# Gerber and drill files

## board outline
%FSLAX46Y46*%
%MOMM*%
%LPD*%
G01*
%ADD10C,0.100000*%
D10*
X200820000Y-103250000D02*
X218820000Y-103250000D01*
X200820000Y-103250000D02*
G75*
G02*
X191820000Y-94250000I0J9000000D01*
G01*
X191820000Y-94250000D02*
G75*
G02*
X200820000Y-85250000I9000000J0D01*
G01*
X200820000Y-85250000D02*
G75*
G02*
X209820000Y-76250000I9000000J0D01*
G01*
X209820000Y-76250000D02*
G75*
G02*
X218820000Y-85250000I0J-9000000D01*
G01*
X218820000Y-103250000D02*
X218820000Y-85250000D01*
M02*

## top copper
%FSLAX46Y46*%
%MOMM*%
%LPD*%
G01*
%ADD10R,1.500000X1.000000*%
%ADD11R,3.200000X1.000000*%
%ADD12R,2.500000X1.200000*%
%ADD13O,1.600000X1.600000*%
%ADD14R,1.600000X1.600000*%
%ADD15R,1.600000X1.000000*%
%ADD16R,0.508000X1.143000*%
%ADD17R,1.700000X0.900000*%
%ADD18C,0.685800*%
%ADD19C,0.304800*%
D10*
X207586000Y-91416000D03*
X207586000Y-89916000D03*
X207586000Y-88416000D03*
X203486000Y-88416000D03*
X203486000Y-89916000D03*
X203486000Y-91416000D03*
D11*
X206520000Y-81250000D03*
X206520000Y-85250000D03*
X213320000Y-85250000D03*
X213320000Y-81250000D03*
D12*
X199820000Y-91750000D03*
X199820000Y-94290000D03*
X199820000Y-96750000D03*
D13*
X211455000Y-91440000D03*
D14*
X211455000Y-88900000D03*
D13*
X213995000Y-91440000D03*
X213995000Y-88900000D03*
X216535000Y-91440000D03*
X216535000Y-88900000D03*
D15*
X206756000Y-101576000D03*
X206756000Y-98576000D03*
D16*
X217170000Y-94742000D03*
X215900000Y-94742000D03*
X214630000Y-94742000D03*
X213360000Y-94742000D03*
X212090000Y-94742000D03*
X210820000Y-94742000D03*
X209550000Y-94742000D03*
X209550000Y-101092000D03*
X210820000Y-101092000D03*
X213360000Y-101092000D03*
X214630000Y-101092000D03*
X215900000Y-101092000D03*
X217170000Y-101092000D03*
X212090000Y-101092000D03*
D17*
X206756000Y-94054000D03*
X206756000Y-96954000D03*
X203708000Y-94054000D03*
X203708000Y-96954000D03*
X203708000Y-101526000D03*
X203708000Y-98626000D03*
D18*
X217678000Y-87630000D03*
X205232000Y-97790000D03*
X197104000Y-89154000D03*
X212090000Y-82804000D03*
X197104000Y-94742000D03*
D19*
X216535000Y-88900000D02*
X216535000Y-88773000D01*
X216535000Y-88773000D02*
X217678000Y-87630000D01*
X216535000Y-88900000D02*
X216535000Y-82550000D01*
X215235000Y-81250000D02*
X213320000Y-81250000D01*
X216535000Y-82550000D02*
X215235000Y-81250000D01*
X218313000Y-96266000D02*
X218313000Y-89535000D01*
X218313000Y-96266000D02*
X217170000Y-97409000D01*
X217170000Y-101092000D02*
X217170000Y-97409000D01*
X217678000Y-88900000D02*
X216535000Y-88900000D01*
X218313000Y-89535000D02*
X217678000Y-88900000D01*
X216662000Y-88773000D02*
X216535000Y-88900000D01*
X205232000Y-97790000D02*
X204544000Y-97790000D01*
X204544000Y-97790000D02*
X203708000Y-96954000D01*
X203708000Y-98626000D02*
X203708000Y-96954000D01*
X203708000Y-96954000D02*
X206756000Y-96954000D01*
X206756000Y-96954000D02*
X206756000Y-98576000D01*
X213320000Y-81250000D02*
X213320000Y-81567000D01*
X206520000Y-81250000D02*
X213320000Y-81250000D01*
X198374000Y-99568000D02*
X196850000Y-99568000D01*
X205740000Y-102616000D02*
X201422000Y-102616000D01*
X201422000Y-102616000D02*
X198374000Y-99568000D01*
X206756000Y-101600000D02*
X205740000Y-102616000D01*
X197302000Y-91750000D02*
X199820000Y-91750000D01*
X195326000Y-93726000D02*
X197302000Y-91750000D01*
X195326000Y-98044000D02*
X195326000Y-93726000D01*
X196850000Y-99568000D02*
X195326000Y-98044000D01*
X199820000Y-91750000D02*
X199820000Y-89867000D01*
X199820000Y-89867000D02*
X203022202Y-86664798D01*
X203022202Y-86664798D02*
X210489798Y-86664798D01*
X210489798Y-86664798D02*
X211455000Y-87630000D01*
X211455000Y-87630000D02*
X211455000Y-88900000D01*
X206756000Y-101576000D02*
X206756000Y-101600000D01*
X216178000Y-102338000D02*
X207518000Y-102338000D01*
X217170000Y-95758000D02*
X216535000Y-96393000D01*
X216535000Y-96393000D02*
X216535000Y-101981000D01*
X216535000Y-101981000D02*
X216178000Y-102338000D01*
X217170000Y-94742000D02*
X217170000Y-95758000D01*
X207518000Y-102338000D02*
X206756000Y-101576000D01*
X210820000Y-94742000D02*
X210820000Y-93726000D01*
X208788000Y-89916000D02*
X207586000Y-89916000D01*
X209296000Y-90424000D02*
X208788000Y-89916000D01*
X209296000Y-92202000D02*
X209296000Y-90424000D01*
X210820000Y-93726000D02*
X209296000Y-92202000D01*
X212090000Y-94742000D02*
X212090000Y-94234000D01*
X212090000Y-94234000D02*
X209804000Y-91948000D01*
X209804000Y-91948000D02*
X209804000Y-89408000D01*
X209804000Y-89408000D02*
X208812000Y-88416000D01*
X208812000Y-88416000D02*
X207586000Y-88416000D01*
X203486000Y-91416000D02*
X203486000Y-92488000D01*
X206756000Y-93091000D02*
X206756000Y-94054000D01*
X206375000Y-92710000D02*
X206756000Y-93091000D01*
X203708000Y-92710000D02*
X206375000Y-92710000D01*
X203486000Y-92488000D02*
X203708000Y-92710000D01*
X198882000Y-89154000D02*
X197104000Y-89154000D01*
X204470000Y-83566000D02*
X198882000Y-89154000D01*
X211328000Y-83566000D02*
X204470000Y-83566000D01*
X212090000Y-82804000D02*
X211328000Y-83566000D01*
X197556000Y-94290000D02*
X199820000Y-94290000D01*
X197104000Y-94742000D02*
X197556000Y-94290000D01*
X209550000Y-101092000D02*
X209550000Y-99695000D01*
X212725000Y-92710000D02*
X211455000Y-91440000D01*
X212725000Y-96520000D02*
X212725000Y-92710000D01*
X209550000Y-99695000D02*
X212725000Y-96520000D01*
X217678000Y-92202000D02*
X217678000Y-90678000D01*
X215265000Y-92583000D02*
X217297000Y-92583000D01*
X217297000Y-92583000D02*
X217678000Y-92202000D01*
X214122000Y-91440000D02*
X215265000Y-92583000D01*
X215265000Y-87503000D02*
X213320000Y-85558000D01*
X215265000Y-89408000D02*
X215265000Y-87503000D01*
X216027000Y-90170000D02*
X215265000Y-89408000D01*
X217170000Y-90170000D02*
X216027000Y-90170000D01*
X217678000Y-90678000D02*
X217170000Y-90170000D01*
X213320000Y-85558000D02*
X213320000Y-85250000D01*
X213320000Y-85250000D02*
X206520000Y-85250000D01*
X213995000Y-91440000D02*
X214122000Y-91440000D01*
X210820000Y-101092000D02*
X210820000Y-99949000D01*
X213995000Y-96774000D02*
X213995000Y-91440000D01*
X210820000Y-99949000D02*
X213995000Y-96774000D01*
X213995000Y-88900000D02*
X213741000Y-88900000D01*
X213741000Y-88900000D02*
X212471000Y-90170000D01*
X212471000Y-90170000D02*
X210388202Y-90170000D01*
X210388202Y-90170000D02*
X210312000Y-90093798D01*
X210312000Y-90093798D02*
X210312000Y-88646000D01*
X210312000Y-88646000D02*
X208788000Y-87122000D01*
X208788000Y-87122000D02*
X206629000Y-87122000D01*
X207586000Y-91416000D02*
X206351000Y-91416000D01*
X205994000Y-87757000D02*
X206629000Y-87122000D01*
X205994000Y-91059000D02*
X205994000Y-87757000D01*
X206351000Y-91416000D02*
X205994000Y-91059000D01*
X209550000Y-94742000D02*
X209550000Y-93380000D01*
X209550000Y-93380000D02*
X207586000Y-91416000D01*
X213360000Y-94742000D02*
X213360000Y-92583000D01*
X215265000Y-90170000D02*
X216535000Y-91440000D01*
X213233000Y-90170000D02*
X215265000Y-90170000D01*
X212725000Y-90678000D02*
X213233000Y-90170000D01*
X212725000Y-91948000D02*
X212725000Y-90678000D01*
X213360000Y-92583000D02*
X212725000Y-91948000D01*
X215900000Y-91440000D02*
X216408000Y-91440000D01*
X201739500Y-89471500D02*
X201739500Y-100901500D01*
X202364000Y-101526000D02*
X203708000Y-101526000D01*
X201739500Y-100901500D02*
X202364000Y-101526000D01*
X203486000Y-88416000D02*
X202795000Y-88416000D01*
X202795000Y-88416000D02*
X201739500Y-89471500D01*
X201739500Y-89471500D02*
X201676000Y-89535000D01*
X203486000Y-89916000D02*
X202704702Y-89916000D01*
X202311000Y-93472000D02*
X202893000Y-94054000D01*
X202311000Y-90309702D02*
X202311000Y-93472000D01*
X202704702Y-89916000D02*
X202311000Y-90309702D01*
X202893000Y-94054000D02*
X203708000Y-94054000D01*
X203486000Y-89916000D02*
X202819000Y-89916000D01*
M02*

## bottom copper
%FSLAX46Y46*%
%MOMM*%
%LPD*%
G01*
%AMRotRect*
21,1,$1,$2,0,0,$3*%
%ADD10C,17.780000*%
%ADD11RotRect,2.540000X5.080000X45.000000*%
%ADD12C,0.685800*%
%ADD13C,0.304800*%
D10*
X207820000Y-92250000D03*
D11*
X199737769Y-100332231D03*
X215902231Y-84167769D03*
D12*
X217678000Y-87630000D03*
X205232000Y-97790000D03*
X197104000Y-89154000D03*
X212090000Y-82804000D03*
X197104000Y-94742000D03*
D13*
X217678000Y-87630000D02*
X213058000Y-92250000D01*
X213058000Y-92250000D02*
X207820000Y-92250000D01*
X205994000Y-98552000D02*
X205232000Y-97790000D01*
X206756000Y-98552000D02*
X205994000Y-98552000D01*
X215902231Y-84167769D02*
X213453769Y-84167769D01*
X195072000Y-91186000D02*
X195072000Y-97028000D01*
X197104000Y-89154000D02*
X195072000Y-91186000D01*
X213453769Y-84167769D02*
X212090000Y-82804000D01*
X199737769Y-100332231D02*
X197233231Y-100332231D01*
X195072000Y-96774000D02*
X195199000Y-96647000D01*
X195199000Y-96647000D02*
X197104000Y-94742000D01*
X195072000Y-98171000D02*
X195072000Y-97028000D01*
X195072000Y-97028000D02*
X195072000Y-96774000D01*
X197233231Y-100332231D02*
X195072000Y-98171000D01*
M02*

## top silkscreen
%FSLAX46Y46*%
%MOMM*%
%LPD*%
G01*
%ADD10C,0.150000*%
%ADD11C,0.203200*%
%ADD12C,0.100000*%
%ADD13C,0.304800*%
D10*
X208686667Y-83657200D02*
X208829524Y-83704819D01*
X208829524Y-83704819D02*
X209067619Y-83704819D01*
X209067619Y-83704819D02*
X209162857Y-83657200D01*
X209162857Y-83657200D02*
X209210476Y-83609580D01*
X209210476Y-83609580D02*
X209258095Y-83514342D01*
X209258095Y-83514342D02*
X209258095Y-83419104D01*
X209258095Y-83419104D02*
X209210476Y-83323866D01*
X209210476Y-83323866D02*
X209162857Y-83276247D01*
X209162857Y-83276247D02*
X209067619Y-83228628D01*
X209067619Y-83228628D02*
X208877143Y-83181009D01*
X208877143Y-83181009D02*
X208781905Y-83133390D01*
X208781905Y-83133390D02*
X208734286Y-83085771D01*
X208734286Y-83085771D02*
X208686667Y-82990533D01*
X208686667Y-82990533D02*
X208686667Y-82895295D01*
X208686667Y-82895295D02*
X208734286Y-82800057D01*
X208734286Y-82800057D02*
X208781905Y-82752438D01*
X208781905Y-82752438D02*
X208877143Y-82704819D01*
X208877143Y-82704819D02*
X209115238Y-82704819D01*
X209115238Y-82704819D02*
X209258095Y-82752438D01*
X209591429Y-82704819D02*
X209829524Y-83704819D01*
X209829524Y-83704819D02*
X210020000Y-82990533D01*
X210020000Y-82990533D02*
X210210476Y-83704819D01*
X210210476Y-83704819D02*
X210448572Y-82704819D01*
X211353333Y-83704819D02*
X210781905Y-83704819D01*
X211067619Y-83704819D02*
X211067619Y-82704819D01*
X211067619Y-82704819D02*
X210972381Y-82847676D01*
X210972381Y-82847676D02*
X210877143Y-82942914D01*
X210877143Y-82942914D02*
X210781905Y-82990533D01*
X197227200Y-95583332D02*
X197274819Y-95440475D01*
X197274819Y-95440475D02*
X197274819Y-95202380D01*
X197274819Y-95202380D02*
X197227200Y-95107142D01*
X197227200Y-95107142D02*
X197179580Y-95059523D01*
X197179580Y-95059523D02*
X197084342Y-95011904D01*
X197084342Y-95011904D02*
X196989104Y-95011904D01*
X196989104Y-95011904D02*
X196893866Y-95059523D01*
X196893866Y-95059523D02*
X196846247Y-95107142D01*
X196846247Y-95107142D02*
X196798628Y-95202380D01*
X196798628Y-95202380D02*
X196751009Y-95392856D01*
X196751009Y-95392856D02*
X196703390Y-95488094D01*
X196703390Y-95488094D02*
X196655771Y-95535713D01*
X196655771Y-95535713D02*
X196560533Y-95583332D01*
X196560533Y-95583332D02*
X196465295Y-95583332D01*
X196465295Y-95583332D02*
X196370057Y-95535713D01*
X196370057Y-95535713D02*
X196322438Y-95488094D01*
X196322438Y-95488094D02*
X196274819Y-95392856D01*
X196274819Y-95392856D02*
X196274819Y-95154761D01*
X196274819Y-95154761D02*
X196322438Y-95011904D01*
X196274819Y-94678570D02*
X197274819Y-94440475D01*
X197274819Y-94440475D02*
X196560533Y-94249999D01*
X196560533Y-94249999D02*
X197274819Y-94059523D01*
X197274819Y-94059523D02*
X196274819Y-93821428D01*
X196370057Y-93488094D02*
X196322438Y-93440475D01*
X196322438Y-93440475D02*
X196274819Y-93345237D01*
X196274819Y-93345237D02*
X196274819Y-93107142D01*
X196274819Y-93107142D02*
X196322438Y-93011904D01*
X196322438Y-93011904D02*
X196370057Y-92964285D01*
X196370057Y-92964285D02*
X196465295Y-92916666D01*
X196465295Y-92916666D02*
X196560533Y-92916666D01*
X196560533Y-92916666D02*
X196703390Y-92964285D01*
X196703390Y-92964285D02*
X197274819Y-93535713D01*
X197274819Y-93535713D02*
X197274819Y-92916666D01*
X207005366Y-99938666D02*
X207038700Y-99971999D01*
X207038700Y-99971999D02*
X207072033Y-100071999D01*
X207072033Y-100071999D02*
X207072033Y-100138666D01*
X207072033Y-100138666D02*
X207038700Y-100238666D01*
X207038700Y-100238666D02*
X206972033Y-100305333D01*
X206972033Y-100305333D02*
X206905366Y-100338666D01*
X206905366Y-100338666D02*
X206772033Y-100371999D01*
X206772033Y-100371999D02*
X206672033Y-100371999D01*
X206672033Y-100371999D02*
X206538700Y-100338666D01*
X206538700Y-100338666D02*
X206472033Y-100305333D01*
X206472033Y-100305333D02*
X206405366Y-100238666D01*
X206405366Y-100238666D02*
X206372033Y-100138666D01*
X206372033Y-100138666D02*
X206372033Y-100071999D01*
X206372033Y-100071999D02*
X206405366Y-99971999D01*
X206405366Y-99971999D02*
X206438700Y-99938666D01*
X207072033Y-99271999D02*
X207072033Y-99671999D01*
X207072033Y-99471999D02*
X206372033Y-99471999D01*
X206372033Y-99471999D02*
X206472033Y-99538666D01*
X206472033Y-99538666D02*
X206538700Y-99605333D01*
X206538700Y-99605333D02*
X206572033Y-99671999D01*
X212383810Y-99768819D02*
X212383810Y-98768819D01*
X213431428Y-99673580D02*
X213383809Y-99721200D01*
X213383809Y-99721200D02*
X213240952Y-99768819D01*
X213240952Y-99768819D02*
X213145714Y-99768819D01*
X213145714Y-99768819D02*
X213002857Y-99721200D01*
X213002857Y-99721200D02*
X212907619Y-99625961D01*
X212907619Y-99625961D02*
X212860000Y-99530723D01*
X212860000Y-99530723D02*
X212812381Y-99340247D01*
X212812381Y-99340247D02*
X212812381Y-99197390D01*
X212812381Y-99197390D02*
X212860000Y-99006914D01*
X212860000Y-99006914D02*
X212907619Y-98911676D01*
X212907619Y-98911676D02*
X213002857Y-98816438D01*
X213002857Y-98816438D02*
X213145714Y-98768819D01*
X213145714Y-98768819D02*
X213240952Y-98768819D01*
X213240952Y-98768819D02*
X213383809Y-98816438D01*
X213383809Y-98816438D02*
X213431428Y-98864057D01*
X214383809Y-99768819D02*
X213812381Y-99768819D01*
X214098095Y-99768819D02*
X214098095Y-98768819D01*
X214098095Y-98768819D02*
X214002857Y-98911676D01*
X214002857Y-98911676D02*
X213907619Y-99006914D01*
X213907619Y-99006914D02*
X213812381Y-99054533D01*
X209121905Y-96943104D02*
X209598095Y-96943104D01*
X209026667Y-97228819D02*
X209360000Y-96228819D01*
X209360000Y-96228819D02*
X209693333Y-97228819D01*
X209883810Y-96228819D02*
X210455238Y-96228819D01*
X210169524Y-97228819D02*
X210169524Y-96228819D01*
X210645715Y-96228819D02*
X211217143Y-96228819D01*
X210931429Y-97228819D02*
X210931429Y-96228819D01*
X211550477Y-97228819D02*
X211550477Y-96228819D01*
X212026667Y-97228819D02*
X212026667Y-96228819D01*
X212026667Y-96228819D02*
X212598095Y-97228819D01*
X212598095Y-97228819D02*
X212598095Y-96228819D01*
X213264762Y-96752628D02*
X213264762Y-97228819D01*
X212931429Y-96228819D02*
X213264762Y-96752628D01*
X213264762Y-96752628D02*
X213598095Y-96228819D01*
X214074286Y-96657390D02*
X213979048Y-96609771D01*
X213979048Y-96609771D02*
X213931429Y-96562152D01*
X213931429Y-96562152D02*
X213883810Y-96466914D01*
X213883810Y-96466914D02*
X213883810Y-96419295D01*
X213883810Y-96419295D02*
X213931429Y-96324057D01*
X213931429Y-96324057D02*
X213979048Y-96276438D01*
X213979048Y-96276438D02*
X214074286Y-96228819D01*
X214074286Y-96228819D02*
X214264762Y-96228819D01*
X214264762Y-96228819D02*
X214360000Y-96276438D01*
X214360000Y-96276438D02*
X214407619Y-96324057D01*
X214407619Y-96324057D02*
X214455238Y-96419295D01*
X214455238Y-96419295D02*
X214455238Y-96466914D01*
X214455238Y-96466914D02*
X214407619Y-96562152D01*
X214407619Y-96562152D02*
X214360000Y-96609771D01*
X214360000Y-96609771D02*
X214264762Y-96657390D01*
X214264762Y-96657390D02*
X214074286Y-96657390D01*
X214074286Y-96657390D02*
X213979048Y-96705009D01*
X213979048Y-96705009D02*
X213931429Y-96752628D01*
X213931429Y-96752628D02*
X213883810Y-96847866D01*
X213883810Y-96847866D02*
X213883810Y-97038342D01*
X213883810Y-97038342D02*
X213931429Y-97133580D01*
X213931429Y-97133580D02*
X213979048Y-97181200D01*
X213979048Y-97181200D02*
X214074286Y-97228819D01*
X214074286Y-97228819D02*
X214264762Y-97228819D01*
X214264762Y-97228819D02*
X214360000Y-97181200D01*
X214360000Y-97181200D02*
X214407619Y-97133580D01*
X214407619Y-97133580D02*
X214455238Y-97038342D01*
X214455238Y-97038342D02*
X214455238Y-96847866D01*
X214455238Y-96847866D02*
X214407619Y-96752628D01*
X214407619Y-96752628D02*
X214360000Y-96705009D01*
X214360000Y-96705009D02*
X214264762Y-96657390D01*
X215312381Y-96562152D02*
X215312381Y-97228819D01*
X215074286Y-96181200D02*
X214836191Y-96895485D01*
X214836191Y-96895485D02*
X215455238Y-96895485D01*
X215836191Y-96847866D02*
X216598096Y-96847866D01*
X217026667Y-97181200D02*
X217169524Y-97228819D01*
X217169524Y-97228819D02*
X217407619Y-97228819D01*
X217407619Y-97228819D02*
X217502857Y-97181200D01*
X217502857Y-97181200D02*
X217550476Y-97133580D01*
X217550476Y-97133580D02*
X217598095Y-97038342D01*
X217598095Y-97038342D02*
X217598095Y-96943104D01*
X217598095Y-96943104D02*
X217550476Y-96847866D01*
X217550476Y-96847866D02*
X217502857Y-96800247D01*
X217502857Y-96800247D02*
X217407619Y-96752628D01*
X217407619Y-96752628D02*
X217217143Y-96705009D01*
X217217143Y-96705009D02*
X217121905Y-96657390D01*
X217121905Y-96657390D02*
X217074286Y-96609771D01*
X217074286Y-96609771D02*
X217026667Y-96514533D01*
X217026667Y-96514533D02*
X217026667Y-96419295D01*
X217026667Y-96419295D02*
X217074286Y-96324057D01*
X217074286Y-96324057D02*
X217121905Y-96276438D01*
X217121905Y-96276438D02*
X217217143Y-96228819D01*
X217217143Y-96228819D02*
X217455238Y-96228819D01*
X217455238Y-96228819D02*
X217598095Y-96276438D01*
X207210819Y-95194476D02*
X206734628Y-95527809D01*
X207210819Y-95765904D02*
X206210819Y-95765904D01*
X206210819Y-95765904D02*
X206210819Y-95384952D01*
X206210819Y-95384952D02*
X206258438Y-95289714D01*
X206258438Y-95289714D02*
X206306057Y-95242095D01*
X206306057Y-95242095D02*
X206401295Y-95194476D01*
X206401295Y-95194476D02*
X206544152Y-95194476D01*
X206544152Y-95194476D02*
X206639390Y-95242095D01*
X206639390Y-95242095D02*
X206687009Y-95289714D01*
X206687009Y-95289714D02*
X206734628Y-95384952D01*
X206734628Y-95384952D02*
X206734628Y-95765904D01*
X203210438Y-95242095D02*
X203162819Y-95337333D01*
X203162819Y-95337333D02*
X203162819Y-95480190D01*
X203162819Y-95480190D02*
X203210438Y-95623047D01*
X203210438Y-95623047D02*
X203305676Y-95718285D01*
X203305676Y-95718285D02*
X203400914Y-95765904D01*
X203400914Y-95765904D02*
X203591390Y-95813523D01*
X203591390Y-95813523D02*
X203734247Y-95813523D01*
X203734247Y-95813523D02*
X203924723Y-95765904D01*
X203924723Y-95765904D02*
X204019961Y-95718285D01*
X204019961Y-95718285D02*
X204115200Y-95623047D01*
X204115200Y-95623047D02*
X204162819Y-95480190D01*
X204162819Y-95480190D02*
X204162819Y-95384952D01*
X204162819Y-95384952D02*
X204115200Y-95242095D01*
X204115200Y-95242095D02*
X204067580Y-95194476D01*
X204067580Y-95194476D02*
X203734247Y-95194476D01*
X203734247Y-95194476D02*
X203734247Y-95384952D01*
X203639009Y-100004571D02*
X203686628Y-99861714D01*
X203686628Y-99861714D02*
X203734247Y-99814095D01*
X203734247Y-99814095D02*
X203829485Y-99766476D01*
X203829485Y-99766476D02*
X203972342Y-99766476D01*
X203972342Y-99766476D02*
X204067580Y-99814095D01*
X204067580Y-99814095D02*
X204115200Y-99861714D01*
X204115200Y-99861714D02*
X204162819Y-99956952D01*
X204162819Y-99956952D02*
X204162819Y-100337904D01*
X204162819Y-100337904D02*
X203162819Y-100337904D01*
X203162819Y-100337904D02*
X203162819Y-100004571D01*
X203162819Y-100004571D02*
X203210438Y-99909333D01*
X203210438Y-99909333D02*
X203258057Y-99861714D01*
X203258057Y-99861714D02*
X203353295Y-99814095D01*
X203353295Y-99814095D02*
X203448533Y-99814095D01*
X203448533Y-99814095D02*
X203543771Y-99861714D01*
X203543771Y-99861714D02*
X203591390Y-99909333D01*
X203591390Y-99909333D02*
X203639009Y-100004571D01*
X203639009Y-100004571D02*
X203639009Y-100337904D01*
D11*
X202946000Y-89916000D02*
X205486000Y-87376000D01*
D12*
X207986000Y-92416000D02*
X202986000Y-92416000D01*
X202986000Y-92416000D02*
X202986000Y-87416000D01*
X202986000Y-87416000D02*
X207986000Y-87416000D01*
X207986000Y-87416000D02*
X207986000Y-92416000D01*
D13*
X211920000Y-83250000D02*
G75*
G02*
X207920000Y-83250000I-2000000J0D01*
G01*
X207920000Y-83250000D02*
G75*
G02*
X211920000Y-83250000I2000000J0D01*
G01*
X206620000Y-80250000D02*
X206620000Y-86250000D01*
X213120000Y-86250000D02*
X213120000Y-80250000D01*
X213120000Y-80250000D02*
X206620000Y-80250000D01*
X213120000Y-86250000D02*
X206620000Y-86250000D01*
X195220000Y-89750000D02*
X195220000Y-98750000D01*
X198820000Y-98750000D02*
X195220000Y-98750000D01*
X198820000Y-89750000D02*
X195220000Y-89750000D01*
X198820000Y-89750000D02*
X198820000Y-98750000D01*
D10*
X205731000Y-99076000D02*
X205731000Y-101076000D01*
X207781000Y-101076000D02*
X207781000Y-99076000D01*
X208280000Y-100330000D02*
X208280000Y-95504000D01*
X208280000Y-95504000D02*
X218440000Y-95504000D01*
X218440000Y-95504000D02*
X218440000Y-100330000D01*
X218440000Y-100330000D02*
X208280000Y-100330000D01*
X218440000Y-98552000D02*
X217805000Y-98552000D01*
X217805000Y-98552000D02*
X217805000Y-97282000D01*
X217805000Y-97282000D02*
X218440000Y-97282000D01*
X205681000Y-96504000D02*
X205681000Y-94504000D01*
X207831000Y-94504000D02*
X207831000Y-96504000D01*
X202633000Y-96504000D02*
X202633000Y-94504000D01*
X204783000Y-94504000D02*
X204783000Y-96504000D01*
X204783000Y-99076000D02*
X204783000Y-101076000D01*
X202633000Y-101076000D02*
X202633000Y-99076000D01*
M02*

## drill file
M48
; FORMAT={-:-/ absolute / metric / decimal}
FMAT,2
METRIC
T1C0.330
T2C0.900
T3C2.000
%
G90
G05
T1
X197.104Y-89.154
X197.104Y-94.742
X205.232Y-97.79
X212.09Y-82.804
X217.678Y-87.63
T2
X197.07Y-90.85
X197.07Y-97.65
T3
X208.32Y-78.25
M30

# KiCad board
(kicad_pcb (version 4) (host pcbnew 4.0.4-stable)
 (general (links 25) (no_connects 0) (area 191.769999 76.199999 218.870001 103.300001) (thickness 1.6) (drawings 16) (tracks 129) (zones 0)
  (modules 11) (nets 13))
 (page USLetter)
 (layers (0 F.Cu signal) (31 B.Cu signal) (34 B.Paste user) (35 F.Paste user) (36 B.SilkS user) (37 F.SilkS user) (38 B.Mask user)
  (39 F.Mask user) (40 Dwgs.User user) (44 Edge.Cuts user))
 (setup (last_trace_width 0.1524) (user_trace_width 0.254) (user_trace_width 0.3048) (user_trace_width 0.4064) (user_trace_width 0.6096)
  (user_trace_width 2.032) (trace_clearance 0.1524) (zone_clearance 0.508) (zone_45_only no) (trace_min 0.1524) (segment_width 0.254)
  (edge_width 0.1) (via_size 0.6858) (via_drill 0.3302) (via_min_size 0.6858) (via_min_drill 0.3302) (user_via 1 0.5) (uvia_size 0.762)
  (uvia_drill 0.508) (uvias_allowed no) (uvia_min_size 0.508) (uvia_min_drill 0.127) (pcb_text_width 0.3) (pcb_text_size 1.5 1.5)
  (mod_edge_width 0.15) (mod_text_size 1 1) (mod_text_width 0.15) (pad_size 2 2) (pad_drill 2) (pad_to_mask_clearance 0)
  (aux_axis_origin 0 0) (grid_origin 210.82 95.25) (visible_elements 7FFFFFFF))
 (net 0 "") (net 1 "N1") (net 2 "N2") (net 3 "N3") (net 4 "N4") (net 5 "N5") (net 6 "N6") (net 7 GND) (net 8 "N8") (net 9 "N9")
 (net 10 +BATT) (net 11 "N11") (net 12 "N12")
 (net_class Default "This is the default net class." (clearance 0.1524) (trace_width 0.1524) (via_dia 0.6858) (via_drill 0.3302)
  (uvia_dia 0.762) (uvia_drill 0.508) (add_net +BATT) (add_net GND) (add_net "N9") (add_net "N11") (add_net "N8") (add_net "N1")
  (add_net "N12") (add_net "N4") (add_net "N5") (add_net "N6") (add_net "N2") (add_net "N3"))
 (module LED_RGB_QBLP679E (layer F.Cu) (at 205.486 89.916 180)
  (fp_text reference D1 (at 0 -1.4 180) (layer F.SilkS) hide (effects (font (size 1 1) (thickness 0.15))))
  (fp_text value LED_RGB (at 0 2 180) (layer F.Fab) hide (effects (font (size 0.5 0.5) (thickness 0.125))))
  (fp_line (start 2.54 0) (end 0 2.54) (layer F.SilkS) (width 0.2032))
  (fp_line (start -2.5 -2.5) (end 2.5 -2.5) (layer F.SilkS) (width 0.1))
  (fp_line (start 2.5 -2.5) (end 2.5 2.5) (layer F.SilkS) (width 0.1))
  (fp_line (start 2.5 2.5) (end -2.5 2.5) (layer F.SilkS) (width 0.1))
  (fp_line (start -2.5 2.5) (end -2.5 -2.5) (layer F.SilkS) (width 0.1))
  (pad 4 smd rect (at -2.1 -1.5 270) (size 1 1.5) (layers F.Cu F.Paste F.Mask) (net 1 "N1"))
  (pad 5 smd rect (at -2.1 0 270) (size 1 1.5) (layers F.Cu F.Paste F.Mask) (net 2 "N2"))
  (pad 6 smd rect (at -2.1 1.5 270) (size 1 1.5) (layers F.Cu F.Paste F.Mask) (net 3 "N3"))
  (pad 1 smd rect (at 2 1.5 270) (size 1 1.5) (layers F.Cu F.Paste F.Mask) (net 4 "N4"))
  (pad 2 smd rect (at 2 0 270) (size 1 1.5) (layers F.Cu F.Paste F.Mask) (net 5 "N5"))
  (pad 3 smd rect (at 2 -1.5 270) (size 1 1.5) (layers F.Cu F.Paste F.Mask) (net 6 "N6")))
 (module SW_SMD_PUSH (layer F.Cu) (at 213.32 85.25 180)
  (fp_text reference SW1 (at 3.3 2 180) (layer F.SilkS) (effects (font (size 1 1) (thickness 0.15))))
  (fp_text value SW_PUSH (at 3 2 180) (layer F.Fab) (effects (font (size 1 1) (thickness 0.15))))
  (fp_circle (center 3.4 2) (end 3.4 0) (layer F.SilkS) (width 0.3048))
  (fp_line (start 6.7 5) (end 6.7 -1) (layer F.SilkS) (width 0.3048))
  (fp_line (start 0.2 -1) (end 0.2 5) (layer F.SilkS) (width 0.3048))
  (fp_line (start 0.2 5) (end 6.7 5) (layer F.SilkS) (width 0.3048))
  (fp_line (start 0.2 -1) (end 6.7 -1) (layer F.SilkS) (width 0.3048))
  (pad 2 smd rect (at 6.8 4 180) (size 3.2 1) (layers F.Cu F.Paste F.Mask) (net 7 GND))
  (pad 1 smd rect (at 6.8 0 180) (size 3.2 1) (layers F.Cu F.Paste F.Mask) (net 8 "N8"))
  (pad 1 smd rect (at 0 0 180) (size 3.2 1) (layers F.Cu F.Paste F.Mask) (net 8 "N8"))
  (pad 2 smd rect (at 0 4 180) (size 3.2 1) (layers F.Cu F.Paste F.Mask) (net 7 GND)))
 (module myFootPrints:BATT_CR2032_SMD (layer B.Cu) (at 207.82 92.25 45)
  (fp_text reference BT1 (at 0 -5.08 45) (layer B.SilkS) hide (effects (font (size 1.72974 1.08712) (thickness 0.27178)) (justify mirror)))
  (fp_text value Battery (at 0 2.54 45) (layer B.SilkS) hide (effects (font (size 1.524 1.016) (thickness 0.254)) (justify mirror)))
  (pad 2 smd circle (at 0 0 45) (size 17.78 17.78) (layers B.Cu B.Paste B.Mask) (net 7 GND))
  (pad 1 smd rect (at -11.43 0 45) (size 2.54 5.08) (layers B.Cu B.Paste B.Mask) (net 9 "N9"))
  (pad 1 smd rect (at 11.43 0 45) (size 2.54 5.08) (layers B.Cu B.Paste B.Mask) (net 9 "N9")))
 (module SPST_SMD (layer F.Cu) (at 199.82 94.25 270)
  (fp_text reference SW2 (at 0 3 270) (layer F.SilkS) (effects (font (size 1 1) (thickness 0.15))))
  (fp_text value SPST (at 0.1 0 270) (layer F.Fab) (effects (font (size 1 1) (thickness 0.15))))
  (fp_line (start -4.5 4.6) (end 4.5 4.6) (layer F.SilkS) (width 0.3048))
  (fp_line (start 4.5 1) (end 4.5 4.6) (layer F.SilkS) (width 0.3048))
  (fp_line (start -4.5 1) (end -4.5 4.6) (layer F.SilkS) (width 0.3048))
  (fp_line (start -4.5 1) (end 4.5 1) (layer F.SilkS) (width 0.3048))
  (pad "" np_thru_hole circle (at 3.4 2.75 270) (size 0.9 0.9) (drill 0.9) (layers *.Cu *.Mask))
  (pad 1 smd rect (at -2.5 0 270) (size 1.2 2.5) (layers F.Cu F.Paste F.Mask) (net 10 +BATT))
  (pad 2 smd rect (at 0.04 0 270) (size 1.2 2.5) (layers F.Cu F.Paste F.Mask) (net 9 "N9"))
  (pad 3 smd rect (at 2.5 0 270) (size 1.2 2.5) (layers F.Cu F.Paste F.Mask))
  (pad "" np_thru_hole circle (at -3.4 2.75 270) (size 0.9 0.9) (drill 0.9) (layers *.Cu *.Mask)))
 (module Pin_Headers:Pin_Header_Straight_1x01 (layer F.Cu) (at 208.32 78.25)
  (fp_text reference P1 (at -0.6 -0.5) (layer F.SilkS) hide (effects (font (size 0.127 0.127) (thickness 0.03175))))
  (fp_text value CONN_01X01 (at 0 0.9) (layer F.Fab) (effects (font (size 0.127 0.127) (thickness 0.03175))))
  (pad "" np_thru_hole circle (at 0 0) (size 2 2) (drill 2) (layers *.Cu *.Mask)))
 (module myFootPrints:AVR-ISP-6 (layer F.Cu) (at 211.455 91.44 90)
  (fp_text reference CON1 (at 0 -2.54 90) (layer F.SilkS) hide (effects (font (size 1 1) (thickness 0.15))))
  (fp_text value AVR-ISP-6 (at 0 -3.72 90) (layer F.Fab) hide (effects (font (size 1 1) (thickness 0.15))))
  (pad 1 smd oval (at 0 0 90) (size 1.6 1.6) (layers F.Cu F.Paste F.Mask) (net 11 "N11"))
  (pad 2 smd rect (at 2.54 0 90) (size 1.6 1.6) (layers F.Cu F.Paste F.Mask) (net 10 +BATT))
  (pad 3 smd oval (at 0 2.54 90) (size 1.6 1.6) (layers F.Cu F.Paste F.Mask) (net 8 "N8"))
  (pad 4 smd oval (at 2.54 2.54 90) (size 1.6 1.6) (layers F.Cu F.Paste F.Mask) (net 1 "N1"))
  (pad 5 smd oval (at 0 5.08 90) (size 1.6 1.6) (layers F.Cu F.Paste F.Mask) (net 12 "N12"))
  (pad 6 smd oval (at 2.54 5.08 90) (size 1.6 1.6) (layers F.Cu F.Paste F.Mask) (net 7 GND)))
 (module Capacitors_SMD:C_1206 (layer F.Cu) (at 206.756 100.076 90)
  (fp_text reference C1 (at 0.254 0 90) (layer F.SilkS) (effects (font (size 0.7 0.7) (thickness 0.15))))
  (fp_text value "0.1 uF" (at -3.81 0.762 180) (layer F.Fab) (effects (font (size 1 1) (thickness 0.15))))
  (fp_line (start 1 -1.025) (end -1 -1.025) (layer F.SilkS) (width 0.15))
  (fp_line (start -1 1.025) (end 1 1.025) (layer F.SilkS) (width 0.15))
  (pad 1 smd rect (at -1.5 0 90) (size 1 1.6) (layers F.Cu F.Paste F.Mask) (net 10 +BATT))
  (pad 2 smd rect (at 1.5 0 90) (size 1 1.6) (layers F.Cu F.Paste F.Mask) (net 7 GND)))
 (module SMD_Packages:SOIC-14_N (layer F.Cu) (at 213.36 98.044 180)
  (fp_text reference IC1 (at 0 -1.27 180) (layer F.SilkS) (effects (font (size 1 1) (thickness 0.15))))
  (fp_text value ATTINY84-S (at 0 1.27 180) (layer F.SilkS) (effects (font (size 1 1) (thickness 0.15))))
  (fp_line (start 5.08 -2.286) (end 5.08 2.54) (layer F.SilkS) (width 0.15))
  (fp_line (start 5.08 2.54) (end -5.08 2.54) (layer F.SilkS) (width 0.15))
  (fp_line (start -5.08 2.54) (end -5.08 -2.286) (layer F.SilkS) (width 0.15))
  (fp_line (start -5.08 -2.286) (end 5.08 -2.286) (layer F.SilkS) (width 0.15))
  (fp_line (start -5.08 -0.508) (end -4.445 -0.508) (layer F.SilkS) (width 0.15))
  (fp_line (start -4.445 -0.508) (end -4.445 0.762) (layer F.SilkS) (width 0.15))
  (fp_line (start -4.445 0.762) (end -5.08 0.762) (layer F.SilkS) (width 0.15))
  (pad 1 smd rect (at -3.81 3.302 180) (size 0.508 1.143) (layers F.Cu F.Paste F.Mask) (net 10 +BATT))
  (pad 2 smd rect (at -2.54 3.302 180) (size 0.508 1.143) (layers F.Cu F.Paste F.Mask))
  (pad 3 smd rect (at -1.27 3.302 180) (size 0.508 1.143) (layers F.Cu F.Paste F.Mask))
  (pad 4 smd rect (at 0 3.302 180) (size 0.508 1.143) (layers F.Cu F.Paste F.Mask) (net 12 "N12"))
  (pad 5 smd rect (at 1.27 3.302 180) (size 0.508 1.143) (layers F.Cu F.Paste F.Mask) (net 3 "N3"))
  (pad 6 smd rect (at 2.54 3.302 180) (size 0.508 1.143) (layers F.Cu F.Paste F.Mask) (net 2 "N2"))
  (pad 7 smd rect (at 3.81 3.302 180) (size 0.508 1.143) (layers F.Cu F.Paste F.Mask) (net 1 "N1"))
  (pad 8 smd rect (at 3.81 -3.048 180) (size 0.508 1.143) (layers F.Cu F.Paste F.Mask) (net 11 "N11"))
  (pad 9 smd rect (at 2.54 -3.048 180) (size 0.508 1.143) (layers F.Cu F.Paste F.Mask) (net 8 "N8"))
  (pad 11 smd rect (at 0 -3.048 180) (size 0.508 1.143) (layers F.Cu F.Paste F.Mask))
  (pad 12 smd rect (at -1.27 -3.048 180) (size 0.508 1.143) (layers F.Cu F.Paste F.Mask))
  (pad 13 smd rect (at -2.54 -3.048 180) (size 0.508 1.143) (layers F.Cu F.Paste F.Mask))
  (pad 14 smd rect (at -3.81 -3.048 180) (size 0.508 1.143) (layers F.Cu F.Paste F.Mask) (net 7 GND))
  (pad 10 smd rect (at 1.27 -3.048 180) (size 0.508 1.143) (layers F.Cu F.Paste F.Mask)))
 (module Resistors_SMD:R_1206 (layer F.Cu) (at 206.756 95.504 270)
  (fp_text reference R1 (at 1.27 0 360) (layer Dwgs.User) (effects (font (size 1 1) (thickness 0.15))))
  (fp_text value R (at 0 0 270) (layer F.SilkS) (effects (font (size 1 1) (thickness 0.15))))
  (fp_line (start 1 1.075) (end -1 1.075) (layer F.SilkS) (width 0.15))
  (fp_line (start -1 -1.075) (end 1 -1.075) (layer F.SilkS) (width 0.15))
  (pad 1 smd rect (at -1.45 0 270) (size 0.9 1.7) (layers F.Cu F.Paste F.Mask) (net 6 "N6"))
  (pad 2 smd rect (at 1.45 0 270) (size 0.9 1.7) (layers F.Cu F.Paste F.Mask) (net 7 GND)))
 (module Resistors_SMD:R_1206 (layer F.Cu) (at 203.708 95.504 270)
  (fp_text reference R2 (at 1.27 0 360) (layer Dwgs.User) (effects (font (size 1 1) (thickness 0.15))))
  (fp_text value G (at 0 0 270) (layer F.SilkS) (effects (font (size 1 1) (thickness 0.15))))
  (fp_line (start 1 1.075) (end -1 1.075) (layer F.SilkS) (width 0.15))
  (fp_line (start -1 -1.075) (end 1 -1.075) (layer F.SilkS) (width 0.15))
  (pad 1 smd rect (at -1.45 0 270) (size 0.9 1.7) (layers F.Cu F.Paste F.Mask) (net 5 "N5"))
  (pad 2 smd rect (at 1.45 0 270) (size 0.9 1.7) (layers F.Cu F.Paste F.Mask) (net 7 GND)))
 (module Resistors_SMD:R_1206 (layer F.Cu) (at 203.708 100.076 90)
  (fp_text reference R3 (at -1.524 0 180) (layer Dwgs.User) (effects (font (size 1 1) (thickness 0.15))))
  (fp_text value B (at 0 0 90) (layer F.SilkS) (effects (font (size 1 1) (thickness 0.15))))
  (fp_line (start 1 1.075) (end -1 1.075) (layer F.SilkS) (width 0.15))
  (fp_line (start -1 -1.075) (end 1 -1.075) (layer F.SilkS) (width 0.15))
  (pad 1 smd rect (at -1.45 0 90) (size 0.9 1.7) (layers F.Cu F.Paste F.Mask) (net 4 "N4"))
  (pad 2 smd rect (at 1.45 0 90) (size 0.9 1.7) (layers F.Cu F.Paste F.Mask) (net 7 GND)))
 (gr_line (start 200.82 103.25) (end 218.82 103.25) (angle 90) (layer Edge.Cuts) (width 0.1))
 (gr_arc (start 200.82 94.25) (end 200.82 103.25) (angle 90) (layer Edge.Cuts) (width 0.1))
 (gr_arc (start 200.82 94.25) (end 191.82 94.25) (angle 90) (layer Edge.Cuts) (width 0.1))
 (gr_arc (start 209.82 85.25) (end 200.82 85.25) (angle 90) (layer Edge.Cuts) (width 0.1))
 (gr_arc (start 209.82 85.25) (end 209.82 76.25) (angle 90) (layer Edge.Cuts) (width 0.1))
 (gr_line (start 218.82 103.25) (end 218.82 85.25) (angle 90) (layer Edge.Cuts) (width 0.1))
 (segment (start 216.535 88.9) (end 216.535 88.773) (width 0.3048) (layer F.Cu) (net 7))
 (segment (start 216.535 88.773) (end 217.678 87.63) (width 0.3048) (layer F.Cu) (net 7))
 (segment (start 217.678 87.63) (end 213.058 92.25) (width 0.3048) (layer B.Cu) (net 7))
 (via (at 217.678 87.63) (size 0.6858) (drill 0.3302) (layers F.Cu B.Cu) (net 7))
 (segment (start 213.058 92.25) (end 207.82 92.25) (width 0.3048) (layer B.Cu) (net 7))
 (segment (start 216.535 88.9) (end 216.535 82.55) (width 0.3048) (layer F.Cu) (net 7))
 (segment (start 215.235 81.25) (end 213.32 81.25) (width 0.3048) (layer F.Cu) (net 7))
 (segment (start 216.535 82.55) (end 215.235 81.25) (width 0.3048) (layer F.Cu) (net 7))
 (segment (start 218.313 96.266) (end 218.313 89.535) (width 0.3048) (layer F.Cu) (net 7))
 (segment (start 218.313 96.266) (end 217.17 97.409) (width 0.3048) (layer F.Cu) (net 7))
 (segment (start 217.17 101.092) (end 217.17 97.409) (width 0.3048) (layer F.Cu) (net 7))
 (segment (start 217.678 88.9) (end 216.535 88.9) (width 0.3048) (layer F.Cu) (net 7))
 (segment (start 218.313 89.535) (end 217.678 88.9) (width 0.3048) (layer F.Cu) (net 7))
 (segment (start 216.662 88.773) (end 216.535 88.9) (width 0.3048) (layer F.Cu) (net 7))
 (segment (start 205.232 97.79) (end 204.544 97.79) (width 0.3048) (layer F.Cu) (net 7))
 (segment (start 205.994 98.552) (end 205.232 97.79) (width 0.3048) (layer B.Cu) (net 7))
 (via (at 205.232 97.79) (size 0.6858) (drill 0.3302) (layers F.Cu B.Cu) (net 7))
 (segment (start 204.544 97.79) (end 203.708 96.954) (width 0.3048) (layer F.Cu) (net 7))
 (segment (start 206.756 98.552) (end 205.994 98.552) (width 0.3048) (layer B.Cu) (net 7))
 (segment (start 203.708 98.626) (end 203.708 96.954) (width 0.3048) (layer F.Cu) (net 7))
 (segment (start 203.708 96.954) (end 206.756 96.954) (width 0.3048) (layer F.Cu) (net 7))
 (segment (start 206.756 96.954) (end 206.756 98.576) (width 0.3048) (layer F.Cu) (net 7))
 (segment (start 213.32 81.25) (end 213.32 81.567) (width 0.3048) (layer F.Cu) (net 7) (status 30))
 (segment (start 206.52 81.25) (end 213.32 81.25) (width 0.3048) (layer F.Cu) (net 7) (status 30))
 (segment (start 198.374 99.568) (end 196.85 99.568) (width 0.3048) (layer F.Cu) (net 10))
 (segment (start 205.74 102.616) (end 201.422 102.616) (width 0.3048) (layer F.Cu) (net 10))
 (segment (start 201.422 102.616) (end 198.374 99.568) (width 0.3048) (layer F.Cu) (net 10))
 (segment (start 206.756 101.6) (end 205.74 102.616) (width 0.3048) (layer F.Cu) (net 10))
 (segment (start 197.302 91.75) (end 199.82 91.75) (width 0.3048) (layer F.Cu) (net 10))
 (segment (start 195.326 93.726) (end 197.302 91.75) (width 0.3048) (layer F.Cu) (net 10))
 (segment (start 195.326 98.044) (end 195.326 93.726) (width 0.3048) (layer F.Cu) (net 10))
 (segment (start 196.85 99.568) (end 195.326 98.044) (width 0.3048) (layer F.Cu) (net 10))
 (segment (start 199.82 91.75) (end 199.82 89.867) (width 0.3048) (layer F.Cu) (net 10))
 (segment (start 199.82 89.867) (end 203.022202 86.664798) (width 0.3048) (layer F.Cu) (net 10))
 (segment (start 203.022202 86.664798) (end 210.489798 86.664798) (width 0.3048) (layer F.Cu) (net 10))
 (segment (start 210.489798 86.664798) (end 211.455 87.63) (width 0.3048) (layer F.Cu) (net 10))
 (segment (start 211.455 87.63) (end 211.455 88.9) (width 0.3048) (layer F.Cu) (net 10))
 (segment (start 206.756 101.576) (end 206.756 101.6) (width 0.3048) (layer F.Cu) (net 10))
 (segment (start 216.178 102.338) (end 207.518 102.338) (width 0.3048) (layer F.Cu) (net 10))
 (segment (start 217.17 95.758) (end 216.535 96.393) (width 0.3048) (layer F.Cu) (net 10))
 (segment (start 216.535 96.393) (end 216.535 101.981) (width 0.3048) (layer F.Cu) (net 10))
 (segment (start 216.535 101.981) (end 216.178 102.338) (width 0.3048) (layer F.Cu) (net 10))
 (segment (start 217.17 94.742) (end 217.17 95.758) (width 0.3048) (layer F.Cu) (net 10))
 (segment (start 207.518 102.338) (end 206.756 101.576) (width 0.3048) (layer F.Cu) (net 10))
 (segment (start 210.82 94.742) (end 210.82 93.726) (width 0.3048) (layer F.Cu) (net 2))
 (segment (start 208.788 89.916) (end 207.586 89.916) (width 0.3048) (layer F.Cu) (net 2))
 (segment (start 209.296 90.424) (end 208.788 89.916) (width 0.3048) (layer F.Cu) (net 2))
 (segment (start 209.296 92.202) (end 209.296 90.424) (width 0.3048) (layer F.Cu) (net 2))
 (segment (start 210.82 93.726) (end 209.296 92.202) (width 0.3048) (layer F.Cu) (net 2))
 (segment (start 212.09 94.742) (end 212.09 94.234) (width 0.3048) (layer F.Cu) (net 3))
 (segment (start 212.09 94.234) (end 209.804 91.948) (width 0.3048) (layer F.Cu) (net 3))
 (segment (start 209.804 91.948) (end 209.804 89.408) (width 0.3048) (layer F.Cu) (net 3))
 (segment (start 209.804 89.408) (end 208.812 88.416) (width 0.3048) (layer F.Cu) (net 3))
 (segment (start 208.812 88.416) (end 207.586 88.416) (width 0.3048) (layer F.Cu) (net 3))
 (segment (start 203.486 91.416) (end 203.486 92.488) (width 0.3048) (layer F.Cu) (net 6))
 (segment (start 206.756 93.091) (end 206.756 94.054) (width 0.3048) (layer F.Cu) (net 6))
 (segment (start 206.375 92.71) (end 206.756 93.091) (width 0.3048) (layer F.Cu) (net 6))
 (segment (start 203.708 92.71) (end 206.375 92.71) (width 0.3048) (layer F.Cu) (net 6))
 (segment (start 203.486 92.488) (end 203.708 92.71) (width 0.3048) (layer F.Cu) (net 6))
 (segment (start 215.902231 84.167769) (end 213.453769 84.167769) (width 0.3048) (layer B.Cu) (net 9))
 (segment (start 195.072 91.186) (end 195.072 97.028) (width 0.3048) (layer B.Cu) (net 9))
 (segment (start 197.104 89.154) (end 195.072 91.186) (width 0.3048) (layer B.Cu) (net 9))
 (via (at 197.104 89.154) (size 0.6858) (drill 0.3302) (layers F.Cu B.Cu) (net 9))
 (segment (start 198.882 89.154) (end 197.104 89.154) (width 0.3048) (layer F.Cu) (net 9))
 (segment (start 204.47 83.566) (end 198.882 89.154) (width 0.3048) (layer F.Cu) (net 9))
 (segment (start 211.328 83.566) (end 204.47 83.566) (width 0.3048) (layer F.Cu) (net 9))
 (segment (start 212.09 82.804) (end 211.328 83.566) (width 0.3048) (layer F.Cu) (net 9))
 (via (at 212.09 82.804) (size 0.6858) (drill 0.3302) (layers F.Cu B.Cu) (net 9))
 (segment (start 213.453769 84.167769) (end 212.09 82.804) (width 0.3048) (layer B.Cu) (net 9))
 (segment (start 199.737769 100.332231) (end 197.233231 100.332231) (width 0.3048) (layer B.Cu) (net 9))
 (segment (start 197.556 94.29) (end 199.82 94.29) (width 0.3048) (layer F.Cu) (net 9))
 (segment (start 197.104 94.742) (end 197.556 94.29) (width 0.3048) (layer F.Cu) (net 9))
 (via (at 197.104 94.742) (size 0.6858) (drill 0.3302) (layers F.Cu B.Cu) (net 9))
 (segment (start 195.072 96.774) (end 195.199 96.647) (width 0.3048) (layer B.Cu) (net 9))
 (segment (start 195.199 96.647) (end 197.104 94.742) (width 0.3048) (layer B.Cu) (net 9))
 (segment (start 195.072 98.171) (end 195.072 97.028) (width 0.3048) (layer B.Cu) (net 9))
 (segment (start 195.072 97.028) (end 195.072 96.774) (width 0.3048) (layer B.Cu) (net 9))
 (segment (start 197.233231 100.332231) (end 195.072 98.171) (width 0.3048) (layer B.Cu) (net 9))
 (segment (start 209.55 101.092) (end 209.55 99.695) (width 0.3048) (layer F.Cu) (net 11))
 (segment (start 212.725 92.71) (end 211.455 91.44) (width 0.3048) (layer F.Cu) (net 11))
 (segment (start 212.725 96.52) (end 212.725 92.71) (width 0.3048) (layer F.Cu) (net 11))
 (segment (start 209.55 99.695) (end 212.725 96.52) (width 0.3048) (layer F.Cu) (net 11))
 (segment (start 217.678 92.202) (end 217.678 90.678) (width 0.3048) (layer F.Cu) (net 8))
 (segment (start 215.265 92.583) (end 217.297 92.583) (width 0.3048) (layer F.Cu) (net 8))
 (segment (start 217.297 92.583) (end 217.678 92.202) (width 0.3048) (layer F.Cu) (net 8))
 (segment (start 214.122 91.44) (end 215.265 92.583) (width 0.3048) (layer F.Cu) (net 8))
 (segment (start 215.265 87.503) (end 213.32 85.558) (width 0.3048) (layer F.Cu) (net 8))
 (segment (start 215.265 89.408) (end 215.265 87.503) (width 0.3048) (layer F.Cu) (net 8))
 (segment (start 216.027 90.17) (end 215.265 89.408) (width 0.3048) (layer F.Cu) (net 8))
 (segment (start 217.17 90.17) (end 216.027 90.17) (width 0.3048) (layer F.Cu) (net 8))
 (segment (start 217.678 90.678) (end 217.17 90.17) (width 0.3048) (layer F.Cu) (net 8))
 (segment (start 213.32 85.558) (end 213.32 85.25) (width 0.3048) (layer F.Cu) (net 8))
 (segment (start 213.32 85.25) (end 206.52 85.25) (width 0.3048) (layer F.Cu) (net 8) (status 30))
 (segment (start 213.995 91.44) (end 214.122 91.44) (width 0.3048) (layer F.Cu) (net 8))
 (segment (start 210.82 101.092) (end 210.82 99.949) (width 0.3048) (layer F.Cu) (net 8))
 (segment (start 213.995 96.774) (end 213.995 91.44) (width 0.3048) (layer F.Cu) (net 8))
 (segment (start 210.82 99.949) (end 213.995 96.774) (width 0.3048) (layer F.Cu) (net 8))
 (segment (start 213.995 88.9) (end 213.741 88.9) (width 0.3048) (layer F.Cu) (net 1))
 (segment (start 213.741 88.9) (end 212.471 90.17) (width 0.3048) (layer F.Cu) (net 1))
 (segment (start 212.471 90.17) (end 210.388202 90.17) (width 0.3048) (layer F.Cu) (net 1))
 (segment (start 210.388202 90.17) (end 210.312 90.093798) (width 0.3048) (layer F.Cu) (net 1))
 (segment (start 210.312 90.093798) (end 210.312 88.646) (width 0.3048) (layer F.Cu) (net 1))
 (segment (start 210.312 88.646) (end 208.788 87.122) (width 0.3048) (layer F.Cu) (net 1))
 (segment (start 208.788 87.122) (end 206.629 87.122) (width 0.3048) (layer F.Cu) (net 1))
 (segment (start 207.586 91.416) (end 206.351 91.416) (width 0.3048) (layer F.Cu) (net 1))
 (segment (start 205.994 87.757) (end 206.629 87.122) (width 0.3048) (layer F.Cu) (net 1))
 (segment (start 205.994 91.059) (end 205.994 87.757) (width 0.3048) (layer F.Cu) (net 1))
 (segment (start 206.351 91.416) (end 205.994 91.059) (width 0.3048) (layer F.Cu) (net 1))
 (segment (start 209.55 94.742) (end 209.55 93.38) (width 0.3048) (layer F.Cu) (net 1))
 (segment (start 209.55 93.38) (end 207.586 91.416) (width 0.3048) (layer F.Cu) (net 1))
 (segment (start 213.36 94.742) (end 213.36 92.583) (width 0.3048) (layer F.Cu) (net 12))
 (segment (start 215.265 90.17) (end 216.535 91.44) (width 0.3048) (layer F.Cu) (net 12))
 (segment (start 213.233 90.17) (end 215.265 90.17) (width 0.3048) (layer F.Cu) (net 12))
 (segment (start 212.725 90.678) (end 213.233 90.17) (width 0.3048) (layer F.Cu) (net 12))
 (segment (start 212.725 91.948) (end 212.725 90.678) (width 0.3048) (layer F.Cu) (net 12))
 (segment (start 213.36 92.583) (end 212.725 91.948) (width 0.3048) (layer F.Cu) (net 12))
 (segment (start 215.9 91.44) (end 216.408 91.44) (width 0.3048) (layer F.Cu) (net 12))
 (segment (start 201.7395 89.4715) (end 201.7395 100.9015) (width 0.3048) (layer F.Cu) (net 4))
 (segment (start 202.364 101.526) (end 203.708 101.526) (width 0.3048) (layer F.Cu) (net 4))
 (segment (start 201.7395 100.9015) (end 202.364 101.526) (width 0.3048) (layer F.Cu) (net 4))
 (segment (start 203.486 88.416) (end 202.795 88.416) (width 0.3048) (layer F.Cu) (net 4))
 (segment (start 202.795 88.416) (end 201.7395 89.4715) (width 0.3048) (layer F.Cu) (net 4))
 (segment (start 201.7395 89.4715) (end 201.676 89.535) (width 0.3048) (layer F.Cu) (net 4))
 (segment (start 203.486 89.916) (end 202.704702 89.916) (width 0.3048) (layer F.Cu) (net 5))
 (segment (start 202.311 93.472) (end 202.893 94.054) (width 0.3048) (layer F.Cu) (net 5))
 (segment (start 202.311 90.309702) (end 202.311 93.472) (width 0.3048) (layer F.Cu) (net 5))
 (segment (start 202.704702 89.916) (end 202.311 90.309702) (width 0.3048) (layer F.Cu) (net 5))
 (segment (start 202.893 94.054) (end 203.708 94.054) (width 0.3048) (layer F.Cu) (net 5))
 (segment (start 203.486 89.916) (end 202.819 89.916) (width 0.3048) (layer F.Cu) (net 5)))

